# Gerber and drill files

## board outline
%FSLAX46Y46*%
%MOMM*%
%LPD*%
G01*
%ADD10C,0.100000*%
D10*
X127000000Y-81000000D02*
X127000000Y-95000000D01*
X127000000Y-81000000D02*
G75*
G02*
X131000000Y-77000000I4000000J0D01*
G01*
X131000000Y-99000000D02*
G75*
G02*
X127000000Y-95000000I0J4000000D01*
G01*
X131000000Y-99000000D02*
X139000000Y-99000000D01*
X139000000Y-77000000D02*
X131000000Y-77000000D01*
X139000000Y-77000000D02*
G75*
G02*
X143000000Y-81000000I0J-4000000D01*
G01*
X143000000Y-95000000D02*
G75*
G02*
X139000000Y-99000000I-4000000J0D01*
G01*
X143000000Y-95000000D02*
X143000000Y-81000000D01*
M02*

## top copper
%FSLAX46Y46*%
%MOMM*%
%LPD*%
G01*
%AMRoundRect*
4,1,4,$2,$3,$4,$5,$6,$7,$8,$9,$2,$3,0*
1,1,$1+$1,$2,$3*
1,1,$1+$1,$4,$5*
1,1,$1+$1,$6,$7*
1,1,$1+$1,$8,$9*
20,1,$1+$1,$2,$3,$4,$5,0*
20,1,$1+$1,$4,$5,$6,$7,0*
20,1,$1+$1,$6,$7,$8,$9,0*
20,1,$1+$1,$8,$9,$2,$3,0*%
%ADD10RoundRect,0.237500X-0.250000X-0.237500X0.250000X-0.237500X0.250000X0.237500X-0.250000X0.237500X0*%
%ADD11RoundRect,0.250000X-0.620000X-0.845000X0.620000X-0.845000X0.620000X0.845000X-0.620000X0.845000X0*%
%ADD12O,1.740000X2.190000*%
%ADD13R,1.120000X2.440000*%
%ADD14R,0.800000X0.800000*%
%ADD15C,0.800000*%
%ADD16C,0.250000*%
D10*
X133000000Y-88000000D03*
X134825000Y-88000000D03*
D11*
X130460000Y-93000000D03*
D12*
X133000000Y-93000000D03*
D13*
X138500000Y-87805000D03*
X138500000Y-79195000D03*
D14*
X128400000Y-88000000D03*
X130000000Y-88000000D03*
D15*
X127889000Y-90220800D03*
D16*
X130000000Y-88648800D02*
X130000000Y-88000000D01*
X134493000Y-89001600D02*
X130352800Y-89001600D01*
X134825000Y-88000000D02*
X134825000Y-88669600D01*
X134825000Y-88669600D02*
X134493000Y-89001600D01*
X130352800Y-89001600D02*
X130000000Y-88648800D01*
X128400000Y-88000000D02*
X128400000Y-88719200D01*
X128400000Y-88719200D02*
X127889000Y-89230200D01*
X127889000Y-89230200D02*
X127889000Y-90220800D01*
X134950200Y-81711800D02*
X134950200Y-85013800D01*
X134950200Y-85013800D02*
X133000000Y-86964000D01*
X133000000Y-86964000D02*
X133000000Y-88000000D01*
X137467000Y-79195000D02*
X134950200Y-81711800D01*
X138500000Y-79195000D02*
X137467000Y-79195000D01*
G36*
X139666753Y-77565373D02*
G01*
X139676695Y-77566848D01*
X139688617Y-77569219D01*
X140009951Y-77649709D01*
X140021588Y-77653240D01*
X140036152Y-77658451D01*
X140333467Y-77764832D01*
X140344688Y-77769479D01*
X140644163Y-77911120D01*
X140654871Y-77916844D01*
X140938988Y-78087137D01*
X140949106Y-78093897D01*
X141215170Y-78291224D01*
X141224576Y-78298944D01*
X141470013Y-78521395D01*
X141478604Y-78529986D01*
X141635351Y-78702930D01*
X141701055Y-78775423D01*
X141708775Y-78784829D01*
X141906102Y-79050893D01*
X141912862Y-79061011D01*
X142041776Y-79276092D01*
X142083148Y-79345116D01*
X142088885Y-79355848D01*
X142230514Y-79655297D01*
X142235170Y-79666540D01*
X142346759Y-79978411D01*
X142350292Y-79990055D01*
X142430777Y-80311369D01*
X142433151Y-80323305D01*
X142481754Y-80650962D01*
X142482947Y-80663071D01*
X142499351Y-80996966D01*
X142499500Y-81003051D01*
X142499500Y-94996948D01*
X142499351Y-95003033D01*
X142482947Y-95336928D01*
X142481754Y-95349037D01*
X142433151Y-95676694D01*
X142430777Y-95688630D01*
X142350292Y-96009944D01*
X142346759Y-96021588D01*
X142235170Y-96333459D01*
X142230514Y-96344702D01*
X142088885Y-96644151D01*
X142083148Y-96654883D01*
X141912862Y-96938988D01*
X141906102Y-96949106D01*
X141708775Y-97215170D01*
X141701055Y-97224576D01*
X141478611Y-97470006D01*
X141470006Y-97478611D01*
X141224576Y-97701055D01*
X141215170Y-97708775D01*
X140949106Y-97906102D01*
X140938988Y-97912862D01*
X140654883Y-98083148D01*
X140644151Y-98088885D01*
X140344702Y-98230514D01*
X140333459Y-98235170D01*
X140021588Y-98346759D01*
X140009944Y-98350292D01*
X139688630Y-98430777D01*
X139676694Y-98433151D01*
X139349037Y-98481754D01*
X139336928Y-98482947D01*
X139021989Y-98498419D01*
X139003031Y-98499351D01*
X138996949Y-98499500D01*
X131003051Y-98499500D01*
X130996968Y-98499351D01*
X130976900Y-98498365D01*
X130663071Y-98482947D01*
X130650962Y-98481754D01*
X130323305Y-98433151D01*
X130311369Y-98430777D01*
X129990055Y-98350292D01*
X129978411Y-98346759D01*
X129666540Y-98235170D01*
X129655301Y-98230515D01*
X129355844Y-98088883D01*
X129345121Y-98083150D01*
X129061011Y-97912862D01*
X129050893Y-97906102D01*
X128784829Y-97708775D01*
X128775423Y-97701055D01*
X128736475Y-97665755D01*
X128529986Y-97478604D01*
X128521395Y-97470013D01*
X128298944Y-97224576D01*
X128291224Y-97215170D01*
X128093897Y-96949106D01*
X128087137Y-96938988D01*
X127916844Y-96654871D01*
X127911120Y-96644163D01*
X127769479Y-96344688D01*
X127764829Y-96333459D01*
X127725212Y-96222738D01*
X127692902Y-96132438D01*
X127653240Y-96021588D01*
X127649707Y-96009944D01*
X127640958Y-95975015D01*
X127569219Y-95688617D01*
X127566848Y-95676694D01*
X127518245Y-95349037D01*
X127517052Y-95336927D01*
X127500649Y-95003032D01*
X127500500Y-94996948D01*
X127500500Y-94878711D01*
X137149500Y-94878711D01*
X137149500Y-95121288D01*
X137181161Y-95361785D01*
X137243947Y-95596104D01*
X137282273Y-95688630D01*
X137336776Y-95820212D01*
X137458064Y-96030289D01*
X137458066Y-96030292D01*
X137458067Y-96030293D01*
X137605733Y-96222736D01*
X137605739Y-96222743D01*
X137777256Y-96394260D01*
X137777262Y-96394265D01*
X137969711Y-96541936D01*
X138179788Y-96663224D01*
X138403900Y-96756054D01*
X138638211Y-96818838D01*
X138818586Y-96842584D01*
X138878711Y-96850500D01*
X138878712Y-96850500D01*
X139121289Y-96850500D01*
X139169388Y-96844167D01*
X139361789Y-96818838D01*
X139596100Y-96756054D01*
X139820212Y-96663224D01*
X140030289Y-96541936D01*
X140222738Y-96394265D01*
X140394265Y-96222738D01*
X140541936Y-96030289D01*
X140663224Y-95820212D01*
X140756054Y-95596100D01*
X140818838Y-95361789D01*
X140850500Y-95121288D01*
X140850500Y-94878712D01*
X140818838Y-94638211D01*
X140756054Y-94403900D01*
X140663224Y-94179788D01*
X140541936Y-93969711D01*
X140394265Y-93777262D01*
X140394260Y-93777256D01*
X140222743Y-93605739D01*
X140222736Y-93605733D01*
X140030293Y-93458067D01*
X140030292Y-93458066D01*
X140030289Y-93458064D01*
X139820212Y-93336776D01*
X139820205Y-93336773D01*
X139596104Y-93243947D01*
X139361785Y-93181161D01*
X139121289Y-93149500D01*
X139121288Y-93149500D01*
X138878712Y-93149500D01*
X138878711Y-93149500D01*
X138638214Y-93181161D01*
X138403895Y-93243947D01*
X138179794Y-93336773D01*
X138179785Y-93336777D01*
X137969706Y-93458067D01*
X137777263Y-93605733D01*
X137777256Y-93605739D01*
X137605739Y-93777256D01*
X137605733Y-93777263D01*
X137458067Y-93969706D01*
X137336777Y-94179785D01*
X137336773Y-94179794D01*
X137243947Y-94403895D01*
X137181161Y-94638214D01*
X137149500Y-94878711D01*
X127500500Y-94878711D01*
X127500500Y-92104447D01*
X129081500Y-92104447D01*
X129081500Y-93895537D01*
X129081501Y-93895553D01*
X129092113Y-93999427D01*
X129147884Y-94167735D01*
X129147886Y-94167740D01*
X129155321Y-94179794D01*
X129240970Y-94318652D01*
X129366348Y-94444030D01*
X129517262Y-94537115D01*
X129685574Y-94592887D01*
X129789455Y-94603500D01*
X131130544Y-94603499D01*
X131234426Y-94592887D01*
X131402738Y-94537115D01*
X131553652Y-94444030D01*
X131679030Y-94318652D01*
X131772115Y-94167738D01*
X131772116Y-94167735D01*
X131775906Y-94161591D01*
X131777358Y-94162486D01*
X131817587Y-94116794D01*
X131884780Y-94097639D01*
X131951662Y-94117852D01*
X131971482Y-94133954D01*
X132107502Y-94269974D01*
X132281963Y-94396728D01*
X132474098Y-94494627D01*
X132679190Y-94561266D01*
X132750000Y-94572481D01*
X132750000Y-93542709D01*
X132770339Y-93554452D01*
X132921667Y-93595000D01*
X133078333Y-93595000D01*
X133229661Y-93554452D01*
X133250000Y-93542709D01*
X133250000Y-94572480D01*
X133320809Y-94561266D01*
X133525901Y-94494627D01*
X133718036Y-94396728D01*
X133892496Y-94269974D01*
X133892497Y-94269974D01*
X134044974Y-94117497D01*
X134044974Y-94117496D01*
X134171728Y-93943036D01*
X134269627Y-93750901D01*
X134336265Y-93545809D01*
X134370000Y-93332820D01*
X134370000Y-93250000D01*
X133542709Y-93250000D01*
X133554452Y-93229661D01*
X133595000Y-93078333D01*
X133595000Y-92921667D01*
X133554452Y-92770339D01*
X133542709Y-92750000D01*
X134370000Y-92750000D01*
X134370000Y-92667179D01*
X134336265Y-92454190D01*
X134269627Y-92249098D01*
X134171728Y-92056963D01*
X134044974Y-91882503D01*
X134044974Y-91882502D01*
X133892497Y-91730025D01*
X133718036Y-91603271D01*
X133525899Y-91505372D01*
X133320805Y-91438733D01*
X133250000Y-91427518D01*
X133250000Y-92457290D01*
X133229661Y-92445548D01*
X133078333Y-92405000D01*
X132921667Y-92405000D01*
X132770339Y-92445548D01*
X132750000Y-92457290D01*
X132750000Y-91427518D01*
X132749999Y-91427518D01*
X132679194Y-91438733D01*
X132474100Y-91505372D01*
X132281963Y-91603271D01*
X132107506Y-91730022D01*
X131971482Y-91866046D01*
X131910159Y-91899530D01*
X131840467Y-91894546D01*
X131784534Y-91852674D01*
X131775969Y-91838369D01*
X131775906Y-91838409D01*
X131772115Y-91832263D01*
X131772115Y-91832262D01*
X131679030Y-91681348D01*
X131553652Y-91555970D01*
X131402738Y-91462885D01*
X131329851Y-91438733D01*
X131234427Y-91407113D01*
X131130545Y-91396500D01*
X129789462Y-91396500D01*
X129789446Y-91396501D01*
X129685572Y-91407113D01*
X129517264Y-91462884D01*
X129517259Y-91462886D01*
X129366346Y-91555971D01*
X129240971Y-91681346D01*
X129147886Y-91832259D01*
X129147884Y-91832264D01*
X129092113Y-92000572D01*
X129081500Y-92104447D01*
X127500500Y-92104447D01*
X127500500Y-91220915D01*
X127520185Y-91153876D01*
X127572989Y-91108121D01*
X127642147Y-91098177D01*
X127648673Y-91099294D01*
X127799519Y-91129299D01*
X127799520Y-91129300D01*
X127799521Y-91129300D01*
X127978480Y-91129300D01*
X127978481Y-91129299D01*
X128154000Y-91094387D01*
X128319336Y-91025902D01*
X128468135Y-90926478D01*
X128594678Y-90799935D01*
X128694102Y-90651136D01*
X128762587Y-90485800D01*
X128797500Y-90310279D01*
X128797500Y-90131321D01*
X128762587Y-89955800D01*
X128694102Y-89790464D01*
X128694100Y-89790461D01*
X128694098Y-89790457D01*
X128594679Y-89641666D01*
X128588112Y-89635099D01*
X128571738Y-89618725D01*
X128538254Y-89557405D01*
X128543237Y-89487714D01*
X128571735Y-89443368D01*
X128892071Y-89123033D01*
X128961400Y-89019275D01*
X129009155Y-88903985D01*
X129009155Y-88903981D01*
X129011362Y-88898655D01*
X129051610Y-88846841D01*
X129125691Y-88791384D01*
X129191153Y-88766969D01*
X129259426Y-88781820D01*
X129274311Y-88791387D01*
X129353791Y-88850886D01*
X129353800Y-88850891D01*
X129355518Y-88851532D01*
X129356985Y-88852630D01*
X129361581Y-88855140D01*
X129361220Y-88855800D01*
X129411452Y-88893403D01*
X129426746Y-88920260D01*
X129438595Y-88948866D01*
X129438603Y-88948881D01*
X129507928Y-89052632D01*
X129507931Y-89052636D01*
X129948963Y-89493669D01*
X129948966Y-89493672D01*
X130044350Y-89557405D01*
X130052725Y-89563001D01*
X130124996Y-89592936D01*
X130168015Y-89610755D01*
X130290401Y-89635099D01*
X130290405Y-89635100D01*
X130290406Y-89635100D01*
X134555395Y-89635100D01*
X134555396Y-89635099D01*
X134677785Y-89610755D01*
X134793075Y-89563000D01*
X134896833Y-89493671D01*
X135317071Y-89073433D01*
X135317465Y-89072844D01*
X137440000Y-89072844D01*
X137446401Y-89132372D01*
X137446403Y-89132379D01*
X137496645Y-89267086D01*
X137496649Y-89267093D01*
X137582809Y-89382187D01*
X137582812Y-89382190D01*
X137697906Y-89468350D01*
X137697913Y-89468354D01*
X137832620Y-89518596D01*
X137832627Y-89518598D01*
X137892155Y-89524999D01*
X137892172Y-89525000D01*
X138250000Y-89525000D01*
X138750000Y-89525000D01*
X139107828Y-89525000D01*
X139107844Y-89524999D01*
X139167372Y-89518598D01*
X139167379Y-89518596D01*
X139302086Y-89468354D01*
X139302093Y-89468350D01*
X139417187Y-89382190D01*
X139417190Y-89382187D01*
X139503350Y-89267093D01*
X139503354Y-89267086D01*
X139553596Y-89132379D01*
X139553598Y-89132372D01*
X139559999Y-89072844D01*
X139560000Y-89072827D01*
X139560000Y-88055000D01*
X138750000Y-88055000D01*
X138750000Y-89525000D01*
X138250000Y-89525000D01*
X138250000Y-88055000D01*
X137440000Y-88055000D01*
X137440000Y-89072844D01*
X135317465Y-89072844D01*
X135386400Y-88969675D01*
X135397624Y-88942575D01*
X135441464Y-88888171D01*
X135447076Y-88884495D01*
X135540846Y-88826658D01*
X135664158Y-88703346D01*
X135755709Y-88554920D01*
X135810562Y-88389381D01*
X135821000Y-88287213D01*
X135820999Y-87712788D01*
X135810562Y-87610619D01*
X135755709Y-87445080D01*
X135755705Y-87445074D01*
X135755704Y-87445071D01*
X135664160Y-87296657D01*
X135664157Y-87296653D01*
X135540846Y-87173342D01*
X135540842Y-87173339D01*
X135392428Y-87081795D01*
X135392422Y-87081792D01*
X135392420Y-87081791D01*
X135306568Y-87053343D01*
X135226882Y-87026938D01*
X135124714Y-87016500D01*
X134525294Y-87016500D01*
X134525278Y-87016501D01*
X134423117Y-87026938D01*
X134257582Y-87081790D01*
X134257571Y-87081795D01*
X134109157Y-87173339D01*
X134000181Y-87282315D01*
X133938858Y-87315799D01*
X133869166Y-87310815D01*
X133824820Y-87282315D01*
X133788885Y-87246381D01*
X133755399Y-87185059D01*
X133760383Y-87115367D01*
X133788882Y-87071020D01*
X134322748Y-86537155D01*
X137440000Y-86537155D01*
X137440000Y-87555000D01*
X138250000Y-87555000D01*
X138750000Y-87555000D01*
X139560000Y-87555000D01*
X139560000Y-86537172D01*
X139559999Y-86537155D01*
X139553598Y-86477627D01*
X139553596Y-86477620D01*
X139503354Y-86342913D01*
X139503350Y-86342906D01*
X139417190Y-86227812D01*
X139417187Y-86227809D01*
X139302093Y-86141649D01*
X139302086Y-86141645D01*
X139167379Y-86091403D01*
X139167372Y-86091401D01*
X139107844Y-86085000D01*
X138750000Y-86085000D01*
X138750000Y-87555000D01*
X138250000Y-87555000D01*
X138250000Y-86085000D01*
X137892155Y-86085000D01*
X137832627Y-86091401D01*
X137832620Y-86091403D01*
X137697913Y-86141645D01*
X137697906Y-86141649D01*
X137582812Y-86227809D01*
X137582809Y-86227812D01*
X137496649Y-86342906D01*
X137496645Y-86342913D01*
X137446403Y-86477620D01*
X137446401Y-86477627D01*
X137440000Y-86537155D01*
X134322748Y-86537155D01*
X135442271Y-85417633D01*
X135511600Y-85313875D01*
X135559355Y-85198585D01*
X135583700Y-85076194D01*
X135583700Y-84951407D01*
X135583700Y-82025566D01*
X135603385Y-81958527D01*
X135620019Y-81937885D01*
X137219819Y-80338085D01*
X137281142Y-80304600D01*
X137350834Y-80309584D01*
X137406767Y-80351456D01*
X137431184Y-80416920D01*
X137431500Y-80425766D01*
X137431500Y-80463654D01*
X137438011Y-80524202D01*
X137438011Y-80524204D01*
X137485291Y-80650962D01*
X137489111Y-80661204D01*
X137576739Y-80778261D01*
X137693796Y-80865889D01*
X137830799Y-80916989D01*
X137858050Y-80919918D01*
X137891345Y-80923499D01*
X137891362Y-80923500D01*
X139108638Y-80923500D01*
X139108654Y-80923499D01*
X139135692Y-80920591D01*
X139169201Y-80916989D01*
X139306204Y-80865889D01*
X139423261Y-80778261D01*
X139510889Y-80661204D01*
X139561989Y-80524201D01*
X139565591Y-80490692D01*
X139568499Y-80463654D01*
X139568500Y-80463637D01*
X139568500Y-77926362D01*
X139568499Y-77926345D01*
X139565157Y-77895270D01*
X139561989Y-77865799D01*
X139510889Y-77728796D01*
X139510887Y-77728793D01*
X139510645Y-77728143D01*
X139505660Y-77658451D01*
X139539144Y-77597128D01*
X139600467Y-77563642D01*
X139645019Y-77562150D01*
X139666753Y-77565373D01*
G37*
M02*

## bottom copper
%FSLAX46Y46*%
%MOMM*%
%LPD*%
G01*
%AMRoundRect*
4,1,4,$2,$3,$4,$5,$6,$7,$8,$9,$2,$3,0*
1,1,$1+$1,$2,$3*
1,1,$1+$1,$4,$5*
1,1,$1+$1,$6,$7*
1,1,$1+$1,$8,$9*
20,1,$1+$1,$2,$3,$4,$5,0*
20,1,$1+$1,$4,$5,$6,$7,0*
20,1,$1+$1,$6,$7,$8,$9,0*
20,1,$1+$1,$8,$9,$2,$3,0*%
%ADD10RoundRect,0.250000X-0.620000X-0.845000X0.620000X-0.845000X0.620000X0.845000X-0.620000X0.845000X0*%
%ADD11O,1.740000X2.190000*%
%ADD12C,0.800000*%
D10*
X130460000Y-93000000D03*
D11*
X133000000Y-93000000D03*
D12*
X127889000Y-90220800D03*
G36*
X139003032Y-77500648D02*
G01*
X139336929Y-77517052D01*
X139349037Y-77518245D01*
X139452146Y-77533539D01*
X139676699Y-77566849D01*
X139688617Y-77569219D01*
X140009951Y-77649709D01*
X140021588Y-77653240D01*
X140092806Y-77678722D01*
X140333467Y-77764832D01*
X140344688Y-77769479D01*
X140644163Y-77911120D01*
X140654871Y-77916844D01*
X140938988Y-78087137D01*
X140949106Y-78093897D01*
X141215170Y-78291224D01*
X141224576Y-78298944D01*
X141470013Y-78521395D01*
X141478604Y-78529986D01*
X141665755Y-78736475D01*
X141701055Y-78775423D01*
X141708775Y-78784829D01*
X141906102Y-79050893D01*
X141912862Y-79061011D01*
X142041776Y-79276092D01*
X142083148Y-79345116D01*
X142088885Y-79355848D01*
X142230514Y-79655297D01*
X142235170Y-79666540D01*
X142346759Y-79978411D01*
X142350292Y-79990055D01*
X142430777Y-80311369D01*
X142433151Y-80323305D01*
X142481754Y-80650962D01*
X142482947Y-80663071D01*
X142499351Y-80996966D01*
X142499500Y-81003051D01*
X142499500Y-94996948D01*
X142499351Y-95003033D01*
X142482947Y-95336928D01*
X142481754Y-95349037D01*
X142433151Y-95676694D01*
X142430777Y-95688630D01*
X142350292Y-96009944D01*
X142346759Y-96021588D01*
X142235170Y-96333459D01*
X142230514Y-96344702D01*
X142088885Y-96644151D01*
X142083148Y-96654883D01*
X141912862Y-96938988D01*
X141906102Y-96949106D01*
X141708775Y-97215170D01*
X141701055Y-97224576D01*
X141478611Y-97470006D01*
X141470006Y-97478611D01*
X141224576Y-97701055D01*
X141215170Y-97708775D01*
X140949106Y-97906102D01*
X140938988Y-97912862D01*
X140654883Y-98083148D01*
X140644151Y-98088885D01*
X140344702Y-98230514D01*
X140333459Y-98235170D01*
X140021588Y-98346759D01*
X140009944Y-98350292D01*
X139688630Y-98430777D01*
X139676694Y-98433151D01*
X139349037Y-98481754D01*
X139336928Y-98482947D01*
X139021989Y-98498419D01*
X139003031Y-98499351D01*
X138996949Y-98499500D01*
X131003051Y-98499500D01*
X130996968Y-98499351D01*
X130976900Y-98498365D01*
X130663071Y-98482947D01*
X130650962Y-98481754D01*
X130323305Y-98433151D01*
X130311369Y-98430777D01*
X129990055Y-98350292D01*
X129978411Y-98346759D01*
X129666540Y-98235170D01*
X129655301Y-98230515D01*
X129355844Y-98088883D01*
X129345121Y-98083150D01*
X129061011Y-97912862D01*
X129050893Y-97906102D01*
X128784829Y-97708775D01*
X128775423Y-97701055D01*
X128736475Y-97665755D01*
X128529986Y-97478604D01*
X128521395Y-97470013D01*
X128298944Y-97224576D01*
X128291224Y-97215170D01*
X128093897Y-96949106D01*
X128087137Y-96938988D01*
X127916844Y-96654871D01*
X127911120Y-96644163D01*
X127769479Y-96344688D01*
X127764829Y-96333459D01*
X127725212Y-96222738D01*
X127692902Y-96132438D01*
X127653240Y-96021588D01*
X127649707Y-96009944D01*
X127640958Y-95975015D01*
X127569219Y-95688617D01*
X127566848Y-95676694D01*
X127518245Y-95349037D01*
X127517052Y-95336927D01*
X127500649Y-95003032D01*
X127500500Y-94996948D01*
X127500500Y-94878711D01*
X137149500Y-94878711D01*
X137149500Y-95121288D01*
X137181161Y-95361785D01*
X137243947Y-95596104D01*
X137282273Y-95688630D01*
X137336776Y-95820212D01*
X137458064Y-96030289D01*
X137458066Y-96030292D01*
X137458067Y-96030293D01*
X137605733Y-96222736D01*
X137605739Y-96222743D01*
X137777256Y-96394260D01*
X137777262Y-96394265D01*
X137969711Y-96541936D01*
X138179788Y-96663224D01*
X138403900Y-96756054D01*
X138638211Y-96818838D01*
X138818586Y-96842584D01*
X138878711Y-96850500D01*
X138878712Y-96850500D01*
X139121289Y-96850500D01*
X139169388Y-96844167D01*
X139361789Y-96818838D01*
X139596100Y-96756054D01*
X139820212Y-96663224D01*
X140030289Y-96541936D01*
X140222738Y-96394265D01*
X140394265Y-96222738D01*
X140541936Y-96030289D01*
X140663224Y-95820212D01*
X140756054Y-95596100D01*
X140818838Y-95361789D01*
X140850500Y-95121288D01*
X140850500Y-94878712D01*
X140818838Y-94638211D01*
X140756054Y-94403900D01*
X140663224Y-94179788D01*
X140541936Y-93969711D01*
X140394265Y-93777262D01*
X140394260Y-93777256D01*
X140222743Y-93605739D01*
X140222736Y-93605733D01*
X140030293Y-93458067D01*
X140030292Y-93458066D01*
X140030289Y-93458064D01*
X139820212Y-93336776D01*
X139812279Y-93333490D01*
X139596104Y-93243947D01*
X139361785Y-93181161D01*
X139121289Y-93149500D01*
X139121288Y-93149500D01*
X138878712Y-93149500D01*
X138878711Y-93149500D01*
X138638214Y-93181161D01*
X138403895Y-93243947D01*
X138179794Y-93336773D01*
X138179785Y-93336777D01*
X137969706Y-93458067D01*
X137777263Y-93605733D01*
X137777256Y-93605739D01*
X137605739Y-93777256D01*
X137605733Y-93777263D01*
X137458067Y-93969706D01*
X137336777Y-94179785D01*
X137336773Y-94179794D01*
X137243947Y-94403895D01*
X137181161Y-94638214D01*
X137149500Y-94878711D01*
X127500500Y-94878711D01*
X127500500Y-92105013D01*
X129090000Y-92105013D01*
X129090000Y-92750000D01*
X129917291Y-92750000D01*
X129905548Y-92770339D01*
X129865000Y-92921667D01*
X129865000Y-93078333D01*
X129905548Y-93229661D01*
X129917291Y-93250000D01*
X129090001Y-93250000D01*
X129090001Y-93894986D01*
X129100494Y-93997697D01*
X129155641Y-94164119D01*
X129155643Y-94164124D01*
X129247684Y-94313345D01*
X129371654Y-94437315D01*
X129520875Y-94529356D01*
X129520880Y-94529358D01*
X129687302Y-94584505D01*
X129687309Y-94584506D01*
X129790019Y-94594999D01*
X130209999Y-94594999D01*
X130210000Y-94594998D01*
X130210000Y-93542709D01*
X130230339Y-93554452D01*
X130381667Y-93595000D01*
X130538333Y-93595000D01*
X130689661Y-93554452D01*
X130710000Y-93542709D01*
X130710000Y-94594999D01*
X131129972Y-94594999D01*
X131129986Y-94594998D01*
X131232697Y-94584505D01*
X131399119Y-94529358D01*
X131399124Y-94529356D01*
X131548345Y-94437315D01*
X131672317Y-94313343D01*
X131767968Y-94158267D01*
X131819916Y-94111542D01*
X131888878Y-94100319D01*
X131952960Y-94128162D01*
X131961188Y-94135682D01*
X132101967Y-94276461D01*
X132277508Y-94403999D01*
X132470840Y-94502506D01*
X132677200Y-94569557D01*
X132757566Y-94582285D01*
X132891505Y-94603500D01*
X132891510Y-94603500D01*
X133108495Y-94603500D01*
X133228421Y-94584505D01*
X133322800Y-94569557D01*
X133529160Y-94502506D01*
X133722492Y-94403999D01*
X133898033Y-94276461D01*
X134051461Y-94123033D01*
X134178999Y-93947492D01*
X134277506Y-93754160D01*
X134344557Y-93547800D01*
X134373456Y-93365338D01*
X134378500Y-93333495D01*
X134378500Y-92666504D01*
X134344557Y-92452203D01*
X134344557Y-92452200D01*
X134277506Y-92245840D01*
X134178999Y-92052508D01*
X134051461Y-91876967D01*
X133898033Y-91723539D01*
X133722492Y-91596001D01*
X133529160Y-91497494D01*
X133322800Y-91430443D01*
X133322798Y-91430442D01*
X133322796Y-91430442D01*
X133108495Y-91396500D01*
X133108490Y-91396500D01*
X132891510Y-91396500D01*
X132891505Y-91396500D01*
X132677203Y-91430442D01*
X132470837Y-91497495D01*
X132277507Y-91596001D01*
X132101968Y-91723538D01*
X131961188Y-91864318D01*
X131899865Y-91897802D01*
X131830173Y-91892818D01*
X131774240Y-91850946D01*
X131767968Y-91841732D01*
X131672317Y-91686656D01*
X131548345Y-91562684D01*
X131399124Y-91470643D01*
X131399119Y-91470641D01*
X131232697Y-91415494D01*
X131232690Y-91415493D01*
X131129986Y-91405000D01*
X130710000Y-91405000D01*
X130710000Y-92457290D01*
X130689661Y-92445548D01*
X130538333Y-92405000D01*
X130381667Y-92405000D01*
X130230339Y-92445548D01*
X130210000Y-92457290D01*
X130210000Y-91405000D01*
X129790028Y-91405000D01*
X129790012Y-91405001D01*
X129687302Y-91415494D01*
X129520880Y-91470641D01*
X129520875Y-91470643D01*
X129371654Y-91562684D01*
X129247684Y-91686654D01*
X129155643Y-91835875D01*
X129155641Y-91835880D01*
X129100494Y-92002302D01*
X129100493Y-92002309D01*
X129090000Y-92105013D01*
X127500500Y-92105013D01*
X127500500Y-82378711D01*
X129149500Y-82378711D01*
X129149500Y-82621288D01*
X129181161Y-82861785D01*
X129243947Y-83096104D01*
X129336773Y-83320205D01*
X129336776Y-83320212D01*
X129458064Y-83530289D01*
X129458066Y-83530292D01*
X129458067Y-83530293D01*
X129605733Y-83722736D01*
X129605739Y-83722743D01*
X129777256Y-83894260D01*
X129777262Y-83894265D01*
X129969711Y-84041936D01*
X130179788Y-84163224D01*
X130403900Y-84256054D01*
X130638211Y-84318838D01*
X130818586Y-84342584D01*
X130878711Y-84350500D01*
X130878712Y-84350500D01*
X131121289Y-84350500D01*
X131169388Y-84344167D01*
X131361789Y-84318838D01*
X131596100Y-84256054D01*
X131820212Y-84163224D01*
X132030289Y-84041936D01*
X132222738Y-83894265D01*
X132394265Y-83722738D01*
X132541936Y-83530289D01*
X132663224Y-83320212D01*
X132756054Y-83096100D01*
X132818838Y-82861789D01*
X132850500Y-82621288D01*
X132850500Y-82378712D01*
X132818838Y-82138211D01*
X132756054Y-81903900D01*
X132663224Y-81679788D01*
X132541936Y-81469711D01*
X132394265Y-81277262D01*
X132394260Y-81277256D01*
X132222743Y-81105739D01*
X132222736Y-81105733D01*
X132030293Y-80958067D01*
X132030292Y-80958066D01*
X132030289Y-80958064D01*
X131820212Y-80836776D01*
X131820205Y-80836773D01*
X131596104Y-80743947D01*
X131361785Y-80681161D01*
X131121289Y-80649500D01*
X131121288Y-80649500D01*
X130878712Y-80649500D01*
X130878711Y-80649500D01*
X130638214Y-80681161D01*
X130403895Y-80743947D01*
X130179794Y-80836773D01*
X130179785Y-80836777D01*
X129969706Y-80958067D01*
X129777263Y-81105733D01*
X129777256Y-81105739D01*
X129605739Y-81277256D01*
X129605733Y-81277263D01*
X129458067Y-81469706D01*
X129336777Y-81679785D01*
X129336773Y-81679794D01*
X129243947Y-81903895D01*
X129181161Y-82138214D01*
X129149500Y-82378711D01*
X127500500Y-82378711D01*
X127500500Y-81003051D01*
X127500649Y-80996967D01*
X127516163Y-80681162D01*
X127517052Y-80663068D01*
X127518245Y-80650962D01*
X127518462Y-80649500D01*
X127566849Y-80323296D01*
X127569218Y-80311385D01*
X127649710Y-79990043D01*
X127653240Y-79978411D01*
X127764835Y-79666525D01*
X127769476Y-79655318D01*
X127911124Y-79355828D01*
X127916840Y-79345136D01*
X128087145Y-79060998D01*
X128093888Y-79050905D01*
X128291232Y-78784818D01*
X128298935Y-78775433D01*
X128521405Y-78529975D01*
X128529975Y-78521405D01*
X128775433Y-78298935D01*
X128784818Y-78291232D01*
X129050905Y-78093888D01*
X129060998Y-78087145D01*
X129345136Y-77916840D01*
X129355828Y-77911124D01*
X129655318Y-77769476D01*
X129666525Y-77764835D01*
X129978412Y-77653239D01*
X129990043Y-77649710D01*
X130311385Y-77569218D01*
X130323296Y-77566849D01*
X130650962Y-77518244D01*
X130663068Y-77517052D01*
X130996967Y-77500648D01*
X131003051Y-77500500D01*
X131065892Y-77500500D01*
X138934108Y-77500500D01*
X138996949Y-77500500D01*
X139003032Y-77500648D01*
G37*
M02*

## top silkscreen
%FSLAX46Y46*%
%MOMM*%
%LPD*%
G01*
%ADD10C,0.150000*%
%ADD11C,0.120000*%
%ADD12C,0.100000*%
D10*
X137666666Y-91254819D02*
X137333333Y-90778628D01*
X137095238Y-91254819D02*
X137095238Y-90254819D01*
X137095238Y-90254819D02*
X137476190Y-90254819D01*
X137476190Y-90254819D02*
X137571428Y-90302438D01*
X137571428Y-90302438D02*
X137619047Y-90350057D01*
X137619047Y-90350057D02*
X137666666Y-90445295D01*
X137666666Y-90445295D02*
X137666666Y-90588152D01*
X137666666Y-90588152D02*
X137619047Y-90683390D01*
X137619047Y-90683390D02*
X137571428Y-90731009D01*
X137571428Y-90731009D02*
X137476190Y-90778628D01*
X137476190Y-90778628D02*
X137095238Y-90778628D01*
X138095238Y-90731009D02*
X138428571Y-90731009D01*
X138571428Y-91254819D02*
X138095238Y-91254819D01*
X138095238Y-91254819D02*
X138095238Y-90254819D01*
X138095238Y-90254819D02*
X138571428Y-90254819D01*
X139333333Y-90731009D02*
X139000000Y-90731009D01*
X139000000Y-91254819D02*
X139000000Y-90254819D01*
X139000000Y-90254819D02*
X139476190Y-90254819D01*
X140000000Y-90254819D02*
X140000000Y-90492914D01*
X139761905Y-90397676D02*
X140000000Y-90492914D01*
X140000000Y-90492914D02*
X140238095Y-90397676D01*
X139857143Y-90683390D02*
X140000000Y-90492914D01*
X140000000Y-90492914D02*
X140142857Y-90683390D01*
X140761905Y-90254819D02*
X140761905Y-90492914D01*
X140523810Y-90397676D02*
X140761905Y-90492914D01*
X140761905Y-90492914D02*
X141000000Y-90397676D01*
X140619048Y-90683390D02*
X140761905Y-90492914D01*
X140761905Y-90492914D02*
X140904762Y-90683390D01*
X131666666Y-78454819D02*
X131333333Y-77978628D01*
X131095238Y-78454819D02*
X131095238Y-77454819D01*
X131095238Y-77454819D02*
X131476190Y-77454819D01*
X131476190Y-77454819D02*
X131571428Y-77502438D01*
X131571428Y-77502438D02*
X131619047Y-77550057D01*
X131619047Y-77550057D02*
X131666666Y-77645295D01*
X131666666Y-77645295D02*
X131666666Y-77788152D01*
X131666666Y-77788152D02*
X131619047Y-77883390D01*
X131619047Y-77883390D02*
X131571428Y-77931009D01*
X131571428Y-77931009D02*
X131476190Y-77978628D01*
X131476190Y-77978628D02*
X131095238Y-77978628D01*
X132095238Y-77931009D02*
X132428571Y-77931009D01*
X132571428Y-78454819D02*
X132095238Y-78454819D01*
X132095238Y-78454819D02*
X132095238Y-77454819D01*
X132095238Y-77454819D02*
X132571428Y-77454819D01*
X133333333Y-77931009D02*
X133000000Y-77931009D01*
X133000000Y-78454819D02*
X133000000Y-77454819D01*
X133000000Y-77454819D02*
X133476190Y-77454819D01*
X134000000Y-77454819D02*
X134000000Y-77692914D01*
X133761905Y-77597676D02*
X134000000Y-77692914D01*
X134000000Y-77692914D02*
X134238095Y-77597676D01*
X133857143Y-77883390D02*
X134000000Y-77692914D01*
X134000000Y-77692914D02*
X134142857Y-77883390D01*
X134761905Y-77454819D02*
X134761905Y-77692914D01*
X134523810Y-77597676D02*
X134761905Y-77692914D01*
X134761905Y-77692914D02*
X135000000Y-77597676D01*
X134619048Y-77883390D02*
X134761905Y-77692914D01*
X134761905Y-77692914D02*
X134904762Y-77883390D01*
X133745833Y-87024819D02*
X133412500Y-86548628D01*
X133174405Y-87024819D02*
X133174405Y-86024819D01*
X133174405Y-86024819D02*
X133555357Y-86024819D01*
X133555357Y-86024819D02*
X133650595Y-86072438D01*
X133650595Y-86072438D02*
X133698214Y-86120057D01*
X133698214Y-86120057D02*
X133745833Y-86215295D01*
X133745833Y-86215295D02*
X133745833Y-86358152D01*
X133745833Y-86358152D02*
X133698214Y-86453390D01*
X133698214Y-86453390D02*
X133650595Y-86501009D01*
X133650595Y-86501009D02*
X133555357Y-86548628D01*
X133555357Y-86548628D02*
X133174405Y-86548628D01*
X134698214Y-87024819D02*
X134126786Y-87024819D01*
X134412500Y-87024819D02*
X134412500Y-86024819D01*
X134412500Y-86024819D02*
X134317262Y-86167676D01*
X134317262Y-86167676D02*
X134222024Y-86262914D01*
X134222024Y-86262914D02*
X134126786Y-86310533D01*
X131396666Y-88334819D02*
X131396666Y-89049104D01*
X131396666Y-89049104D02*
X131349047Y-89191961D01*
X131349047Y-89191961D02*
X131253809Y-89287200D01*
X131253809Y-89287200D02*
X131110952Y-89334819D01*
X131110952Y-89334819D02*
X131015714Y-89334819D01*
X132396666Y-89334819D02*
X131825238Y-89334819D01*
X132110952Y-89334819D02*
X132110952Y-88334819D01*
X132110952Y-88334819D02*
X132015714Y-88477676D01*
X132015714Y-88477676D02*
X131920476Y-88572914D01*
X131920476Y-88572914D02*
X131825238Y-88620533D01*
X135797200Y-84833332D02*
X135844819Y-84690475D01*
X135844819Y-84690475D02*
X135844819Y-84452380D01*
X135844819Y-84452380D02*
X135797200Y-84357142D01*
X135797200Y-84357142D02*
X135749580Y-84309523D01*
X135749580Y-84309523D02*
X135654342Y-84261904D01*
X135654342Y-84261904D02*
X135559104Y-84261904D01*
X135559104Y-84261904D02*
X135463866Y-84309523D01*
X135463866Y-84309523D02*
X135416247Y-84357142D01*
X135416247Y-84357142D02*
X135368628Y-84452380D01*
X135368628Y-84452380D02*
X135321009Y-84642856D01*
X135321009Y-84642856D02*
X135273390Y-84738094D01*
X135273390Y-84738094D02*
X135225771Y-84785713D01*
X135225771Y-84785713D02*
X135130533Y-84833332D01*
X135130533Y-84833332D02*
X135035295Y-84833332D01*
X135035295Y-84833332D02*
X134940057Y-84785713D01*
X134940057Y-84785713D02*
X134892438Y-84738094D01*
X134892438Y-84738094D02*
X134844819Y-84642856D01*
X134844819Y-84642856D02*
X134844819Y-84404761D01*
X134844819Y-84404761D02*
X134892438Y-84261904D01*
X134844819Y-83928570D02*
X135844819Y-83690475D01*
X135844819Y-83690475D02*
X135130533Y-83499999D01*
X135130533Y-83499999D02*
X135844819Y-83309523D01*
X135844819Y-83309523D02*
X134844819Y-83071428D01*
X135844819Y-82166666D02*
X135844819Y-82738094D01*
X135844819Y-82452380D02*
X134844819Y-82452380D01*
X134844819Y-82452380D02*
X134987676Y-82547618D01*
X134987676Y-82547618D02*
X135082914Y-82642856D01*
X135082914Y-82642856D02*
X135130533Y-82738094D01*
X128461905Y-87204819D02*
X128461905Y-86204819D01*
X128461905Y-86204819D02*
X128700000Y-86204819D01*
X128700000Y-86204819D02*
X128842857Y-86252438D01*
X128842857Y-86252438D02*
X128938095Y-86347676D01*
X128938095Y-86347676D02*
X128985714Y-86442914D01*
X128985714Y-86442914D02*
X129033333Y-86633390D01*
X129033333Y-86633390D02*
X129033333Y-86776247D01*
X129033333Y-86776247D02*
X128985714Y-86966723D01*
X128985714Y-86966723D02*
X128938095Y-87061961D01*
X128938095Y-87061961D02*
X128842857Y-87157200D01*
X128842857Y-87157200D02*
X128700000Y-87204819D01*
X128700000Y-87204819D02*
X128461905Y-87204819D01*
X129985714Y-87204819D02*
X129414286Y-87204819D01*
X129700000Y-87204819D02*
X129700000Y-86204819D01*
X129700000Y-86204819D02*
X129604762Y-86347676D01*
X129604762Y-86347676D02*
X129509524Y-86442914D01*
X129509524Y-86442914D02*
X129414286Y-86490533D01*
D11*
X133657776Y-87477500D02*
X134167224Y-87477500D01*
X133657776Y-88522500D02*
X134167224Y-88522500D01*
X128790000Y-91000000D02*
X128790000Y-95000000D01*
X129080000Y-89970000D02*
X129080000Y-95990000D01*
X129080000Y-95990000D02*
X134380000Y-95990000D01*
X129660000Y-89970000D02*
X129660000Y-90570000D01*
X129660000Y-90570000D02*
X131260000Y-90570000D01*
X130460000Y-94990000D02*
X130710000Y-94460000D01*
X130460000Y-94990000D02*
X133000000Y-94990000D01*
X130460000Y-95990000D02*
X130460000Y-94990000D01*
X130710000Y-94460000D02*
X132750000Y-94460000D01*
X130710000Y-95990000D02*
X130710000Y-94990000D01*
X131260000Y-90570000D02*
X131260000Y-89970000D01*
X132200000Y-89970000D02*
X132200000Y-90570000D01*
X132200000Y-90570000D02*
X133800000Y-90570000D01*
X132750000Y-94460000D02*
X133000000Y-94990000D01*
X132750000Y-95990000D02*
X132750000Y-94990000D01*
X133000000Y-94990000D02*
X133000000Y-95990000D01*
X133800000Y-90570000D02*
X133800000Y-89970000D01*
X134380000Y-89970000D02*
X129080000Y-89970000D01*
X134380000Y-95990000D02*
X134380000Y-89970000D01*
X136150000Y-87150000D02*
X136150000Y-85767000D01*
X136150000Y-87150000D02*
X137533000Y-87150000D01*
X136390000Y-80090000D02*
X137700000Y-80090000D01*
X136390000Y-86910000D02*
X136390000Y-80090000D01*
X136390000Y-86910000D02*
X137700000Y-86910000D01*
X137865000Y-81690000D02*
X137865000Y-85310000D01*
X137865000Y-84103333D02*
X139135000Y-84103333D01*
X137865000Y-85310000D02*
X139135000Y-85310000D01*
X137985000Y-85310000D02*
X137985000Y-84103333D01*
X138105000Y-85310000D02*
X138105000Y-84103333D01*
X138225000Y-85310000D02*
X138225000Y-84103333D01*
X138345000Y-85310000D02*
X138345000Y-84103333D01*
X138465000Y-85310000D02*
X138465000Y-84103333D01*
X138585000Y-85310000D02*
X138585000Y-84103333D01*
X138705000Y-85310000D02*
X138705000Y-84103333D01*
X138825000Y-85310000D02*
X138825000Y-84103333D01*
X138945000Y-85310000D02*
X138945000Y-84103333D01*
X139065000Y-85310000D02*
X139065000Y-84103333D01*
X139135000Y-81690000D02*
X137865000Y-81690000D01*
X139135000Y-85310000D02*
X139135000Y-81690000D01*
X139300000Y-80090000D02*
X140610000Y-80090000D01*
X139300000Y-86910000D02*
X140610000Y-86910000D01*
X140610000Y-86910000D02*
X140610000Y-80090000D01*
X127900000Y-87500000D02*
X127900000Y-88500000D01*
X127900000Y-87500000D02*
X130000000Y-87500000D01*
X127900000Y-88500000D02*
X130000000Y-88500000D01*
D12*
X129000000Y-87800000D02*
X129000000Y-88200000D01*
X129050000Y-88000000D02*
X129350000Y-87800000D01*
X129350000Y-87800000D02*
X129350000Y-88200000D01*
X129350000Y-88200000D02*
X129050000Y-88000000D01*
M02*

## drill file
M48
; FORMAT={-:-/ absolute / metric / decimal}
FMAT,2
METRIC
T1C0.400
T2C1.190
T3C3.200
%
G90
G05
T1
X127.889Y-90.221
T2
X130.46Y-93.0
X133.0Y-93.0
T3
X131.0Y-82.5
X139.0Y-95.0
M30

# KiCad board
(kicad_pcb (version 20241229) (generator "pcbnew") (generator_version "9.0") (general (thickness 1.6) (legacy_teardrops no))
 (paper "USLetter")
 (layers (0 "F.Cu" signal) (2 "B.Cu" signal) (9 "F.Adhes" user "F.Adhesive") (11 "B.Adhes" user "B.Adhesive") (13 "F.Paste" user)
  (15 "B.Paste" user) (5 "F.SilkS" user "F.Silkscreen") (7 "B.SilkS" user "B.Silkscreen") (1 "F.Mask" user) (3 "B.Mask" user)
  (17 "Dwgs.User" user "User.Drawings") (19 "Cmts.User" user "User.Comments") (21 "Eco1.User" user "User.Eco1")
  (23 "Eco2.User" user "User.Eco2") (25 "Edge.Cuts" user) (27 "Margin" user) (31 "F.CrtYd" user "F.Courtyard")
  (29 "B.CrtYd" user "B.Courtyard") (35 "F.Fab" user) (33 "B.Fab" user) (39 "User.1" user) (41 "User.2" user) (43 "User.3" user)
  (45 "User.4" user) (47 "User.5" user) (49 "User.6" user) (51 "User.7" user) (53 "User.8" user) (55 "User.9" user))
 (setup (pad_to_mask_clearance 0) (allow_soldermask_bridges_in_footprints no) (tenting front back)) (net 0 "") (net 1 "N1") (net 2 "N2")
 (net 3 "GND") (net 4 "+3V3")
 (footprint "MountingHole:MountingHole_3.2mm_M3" (layer "F.Cu") (at 139 95)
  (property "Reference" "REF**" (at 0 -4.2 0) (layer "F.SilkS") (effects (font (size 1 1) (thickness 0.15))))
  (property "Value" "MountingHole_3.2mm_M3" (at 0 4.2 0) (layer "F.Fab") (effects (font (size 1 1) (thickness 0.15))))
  (pad "" np_thru_hole circle (at 0 0) (size 3.2 3.2) (drill 3.2) (layers "*.Cu" "*.Mask")))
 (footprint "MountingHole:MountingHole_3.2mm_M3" (layer "F.Cu") (at 131 82.5)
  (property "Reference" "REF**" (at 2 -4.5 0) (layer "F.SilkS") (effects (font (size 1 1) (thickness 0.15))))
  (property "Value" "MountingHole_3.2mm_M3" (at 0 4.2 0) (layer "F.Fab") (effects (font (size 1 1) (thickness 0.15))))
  (pad "" np_thru_hole circle (at 0 0) (size 3.2 3.2) (drill 3.2) (layers "*.Cu" "*.Mask")))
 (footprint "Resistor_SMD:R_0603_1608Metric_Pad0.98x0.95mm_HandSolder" (layer "F.Cu") (at 133.9125 88)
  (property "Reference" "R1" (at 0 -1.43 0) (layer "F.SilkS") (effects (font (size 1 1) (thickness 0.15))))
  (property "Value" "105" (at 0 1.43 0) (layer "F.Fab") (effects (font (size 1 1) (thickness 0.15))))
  (fp_line (start -0.254724 -0.5225) (end 0.254724 -0.5225) (stroke (width 0.12) (type solid)) (layer "F.SilkS"))
  (fp_line (start -0.254724 0.5225) (end 0.254724 0.5225) (stroke (width 0.12) (type solid)) (layer "F.SilkS"))
  (pad "1" smd roundrect (at -0.9125 0) (size 0.975 0.95) (layers "F.Cu" "F.Mask" "F.Paste") (roundrect_rratio 0.25) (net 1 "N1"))
  (pad "2" smd roundrect (at 0.9125 0) (size 0.975 0.95) (layers "F.Cu" "F.Mask" "F.Paste") (roundrect_rratio 0.25) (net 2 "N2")))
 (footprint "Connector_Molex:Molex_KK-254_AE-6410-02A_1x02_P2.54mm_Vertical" (layer "F.Cu") (at 130.46 93)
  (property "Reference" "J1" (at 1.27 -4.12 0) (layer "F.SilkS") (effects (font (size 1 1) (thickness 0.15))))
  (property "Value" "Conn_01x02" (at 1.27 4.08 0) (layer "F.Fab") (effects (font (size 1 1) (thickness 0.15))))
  (fp_line (start -1.67 -2) (end -1.67 2) (stroke (width 0.12) (type solid)) (layer "F.SilkS"))
  (fp_line (start -1.38 -3.03) (end -1.38 2.99) (stroke (width 0.12) (type solid)) (layer "F.SilkS"))
  (fp_line (start -1.38 2.99) (end 3.92 2.99) (stroke (width 0.12) (type solid)) (layer "F.SilkS"))
  (fp_line (start -0.8 -3.03) (end -0.8 -2.43) (stroke (width 0.12) (type solid)) (layer "F.SilkS"))
  (fp_line (start -0.8 -2.43) (end 0.8 -2.43) (stroke (width 0.12) (type solid)) (layer "F.SilkS"))
  (fp_line (start 0 1.99) (end 0.25 1.46) (stroke (width 0.12) (type solid)) (layer "F.SilkS"))
  (fp_line (start 0 1.99) (end 2.54 1.99) (stroke (width 0.12) (type solid)) (layer "F.SilkS"))
  (fp_line (start 0 2.99) (end 0 1.99) (stroke (width 0.12) (type solid)) (layer "F.SilkS"))
  (fp_line (start 0.25 1.46) (end 2.29 1.46) (stroke (width 0.12) (type solid)) (layer "F.SilkS"))
  (fp_line (start 0.25 2.99) (end 0.25 1.99) (stroke (width 0.12) (type solid)) (layer "F.SilkS"))
  (fp_line (start 0.8 -2.43) (end 0.8 -3.03) (stroke (width 0.12) (type solid)) (layer "F.SilkS"))
  (fp_line (start 1.74 -3.03) (end 1.74 -2.43) (stroke (width 0.12) (type solid)) (layer "F.SilkS"))
  (fp_line (start 1.74 -2.43) (end 3.34 -2.43) (stroke (width 0.12) (type solid)) (layer "F.SilkS"))
  (fp_line (start 2.29 1.46) (end 2.54 1.99) (stroke (width 0.12) (type solid)) (layer "F.SilkS"))
  (fp_line (start 2.29 2.99) (end 2.29 1.99) (stroke (width 0.12) (type solid)) (layer "F.SilkS"))
  (fp_line (start 2.54 1.99) (end 2.54 2.99) (stroke (width 0.12) (type solid)) (layer "F.SilkS"))
  (fp_line (start 3.34 -2.43) (end 3.34 -3.03) (stroke (width 0.12) (type solid)) (layer "F.SilkS"))
  (fp_line (start 3.92 -3.03) (end -1.38 -3.03) (stroke (width 0.12) (type solid)) (layer "F.SilkS"))
  (fp_line (start 3.92 2.99) (end 3.92 -3.03) (stroke (width 0.12) (type solid)) (layer "F.SilkS"))
  (pad "1" thru_hole roundrect (at 0 0) (size 1.74 2.19) (drill 1.19) (layers "*.Cu" "*.Mask") (remove_unused_layers no)
   (roundrect_rratio 0.143678) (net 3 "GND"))
  (pad "2" thru_hole oval (at 2.54 0) (size 1.74 2.19) (drill 1.19) (layers "*.Cu" "*.Mask") (remove_unused_layers no) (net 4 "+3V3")))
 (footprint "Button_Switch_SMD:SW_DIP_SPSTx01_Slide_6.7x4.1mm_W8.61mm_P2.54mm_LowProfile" (layer "F.Cu") (at 138.5 83.5 90)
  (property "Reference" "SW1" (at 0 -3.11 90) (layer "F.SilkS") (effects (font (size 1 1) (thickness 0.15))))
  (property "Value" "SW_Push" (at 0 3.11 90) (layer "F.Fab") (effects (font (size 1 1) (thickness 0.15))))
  (fp_line (start -3.65 -2.35) (end -2.267 -2.35) (stroke (width 0.12) (type solid)) (layer "F.SilkS"))
  (fp_line (start -3.65 -2.35) (end -3.65 -0.967) (stroke (width 0.12) (type solid)) (layer "F.SilkS"))
  (fp_line (start 3.41 -2.11) (end 3.41 -0.8) (stroke (width 0.12) (type solid)) (layer "F.SilkS"))
  (fp_line (start -3.41 -2.11) (end 3.41 -2.11) (stroke (width 0.12) (type solid)) (layer "F.SilkS"))
  (fp_line (start -3.41 -2.11) (end -3.41 -0.8) (stroke (width 0.12) (type solid)) (layer "F.SilkS"))
  (fp_line (start 1.81 -0.635) (end -1.81 -0.635) (stroke (width 0.12) (type solid)) (layer "F.SilkS"))
  (fp_line (start -0.603333 -0.635) (end -0.603333 0.635) (stroke (width 0.12) (type solid)) (layer "F.SilkS"))
  (fp_line (start -1.81 -0.635) (end -1.81 0.635) (stroke (width 0.12) (type solid)) (layer "F.SilkS"))
  (fp_line (start -1.81 -0.515) (end -0.603333 -0.515) (stroke (width 0.12) (type solid)) (layer "F.SilkS"))
  (fp_line (start -1.81 -0.395) (end -0.603333 -0.395) (stroke (width 0.12) (type solid)) (layer "F.SilkS"))
  (fp_line (start -1.81 -0.275) (end -0.603333 -0.275) (stroke (width 0.12) (type solid)) (layer "F.SilkS"))
  (fp_line (start -1.81 -0.155) (end -0.603333 -0.155) (stroke (width 0.12) (type solid)) (layer "F.SilkS"))
  (fp_line (start -1.81 -0.035) (end -0.603333 -0.035) (stroke (width 0.12) (type solid)) (layer "F.SilkS"))
  (fp_line (start -1.81 0.085) (end -0.603333 0.085) (stroke (width 0.12) (type solid)) (layer "F.SilkS"))
  (fp_line (start -1.81 0.205) (end -0.603333 0.205) (stroke (width 0.12) (type solid)) (layer "F.SilkS"))
  (fp_line (start -1.81 0.325) (end -0.603333 0.325) (stroke (width 0.12) (type solid)) (layer "F.SilkS"))
  (fp_line (start -1.81 0.445) (end -0.603333 0.445) (stroke (width 0.12) (type solid)) (layer "F.SilkS"))
  (fp_line (start -1.81 0.565) (end -0.603333 0.565) (stroke (width 0.12) (type solid)) (layer "F.SilkS"))
  (fp_line (start 1.81 0.635) (end 1.81 -0.635) (stroke (width 0.12) (type solid)) (layer "F.SilkS"))
  (fp_line (start -1.81 0.635) (end 1.81 0.635) (stroke (width 0.12) (type solid)) (layer "F.SilkS"))
  (fp_line (start 3.41 0.8) (end 3.41 2.11) (stroke (width 0.12) (type solid)) (layer "F.SilkS"))
  (fp_line (start -3.41 0.8) (end -3.41 2.11) (stroke (width 0.12) (type solid)) (layer "F.SilkS"))
  (fp_line (start -3.41 2.11) (end 3.41 2.11) (stroke (width 0.12) (type solid)) (layer "F.SilkS"))
  (pad "1" smd rect (at -4.305 0 90) (size 2.44 1.12) (layers "F.Cu" "F.Mask" "F.Paste") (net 4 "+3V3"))
  (pad "2" smd rect (at 4.305 0 90) (size 2.44 1.12) (layers "F.Cu" "F.Mask" "F.Paste") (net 1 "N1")))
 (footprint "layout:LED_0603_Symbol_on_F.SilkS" (layer "F.Cu") (at 129.2 88)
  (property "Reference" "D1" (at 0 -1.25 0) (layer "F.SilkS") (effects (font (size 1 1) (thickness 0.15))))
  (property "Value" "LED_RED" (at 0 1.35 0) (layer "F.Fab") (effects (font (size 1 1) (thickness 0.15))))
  (fp_line (start -1.3 -0.5) (end -1.3 0.5) (stroke (width 0.12) (type solid)) (layer "F.SilkS"))
  (fp_line (start -1.3 -0.5) (end 0.8 -0.5) (stroke (width 0.12) (type solid)) (layer "F.SilkS"))
  (fp_line (start -1.3 0.5) (end 0.8 0.5) (stroke (width 0.12) (type solid)) (layer "F.SilkS"))
  (fp_line (start -0.2 -0.2) (end -0.2 0.2) (stroke (width 0.1) (type solid)) (layer "F.SilkS"))
  (fp_line (start -0.15 0) (end 0.15 -0.2) (stroke (width 0.1) (type solid)) (layer "F.SilkS"))
  (fp_line (start 0.15 -0.2) (end 0.15 0.2) (stroke (width 0.1) (type solid)) (layer "F.SilkS"))
  (fp_line (start 0.15 0.2) (end -0.15 0) (stroke (width 0.1) (type solid)) (layer "F.SilkS"))
  (pad "1" smd rect (at -0.8 0 180) (size 0.8 0.8) (layers "F.Cu" "F.Mask" "F.Paste") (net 3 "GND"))
  (pad "2" smd rect (at 0.8 0 180) (size 0.8 0.8) (layers "F.Cu" "F.Mask" "F.Paste") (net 2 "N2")))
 (gr_line (start 127 81) (end 127 95) (stroke (width 0.1) (type default)) (layer "Edge.Cuts"))
 (gr_arc (start 127 81) (mid 128.171573 78.171573) (end 131 77) (stroke (width 0.1) (type default)) (layer "Edge.Cuts"))
 (gr_arc (start 131 99) (mid 128.171573 97.828427) (end 127 95) (stroke (width 0.1) (type default)) (layer "Edge.Cuts"))
 (gr_line (start 131 99) (end 139 99) (stroke (width 0.1) (type default)) (layer "Edge.Cuts"))
 (gr_line (start 139 77) (end 131 77) (stroke (width 0.1) (type default)) (layer "Edge.Cuts"))
 (gr_arc (start 139 77) (mid 141.828427 78.171573) (end 143 81) (stroke (width 0.1) (type default)) (layer "Edge.Cuts"))
 (gr_arc (start 143 95) (mid 141.828427 97.828427) (end 139 99) (stroke (width 0.1) (type default)) (layer "Edge.Cuts"))
 (gr_line (start 143 95) (end 143 81) (stroke (width 0.1) (type default)) (layer "Edge.Cuts"))
 (segment (start 130 88.6488) (end 130 88) (width 0.25) (layer "F.Cu") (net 2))
 (segment (start 134.493 89.0016) (end 130.3528 89.0016) (width 0.25) (layer "F.Cu") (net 2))
 (segment (start 134.825 88) (end 134.825 88.6696) (width 0.25) (layer "F.Cu") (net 2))
 (segment (start 134.825 88.6696) (end 134.493 89.0016) (width 0.25) (layer "F.Cu") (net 2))
 (segment (start 130.3528 89.0016) (end 130 88.6488) (width 0.25) (layer "F.Cu") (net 2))
 (segment (start 128.4 88) (end 128.4 88.7192) (width 0.25) (layer "F.Cu") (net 3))
 (segment (start 128.4 88.7192) (end 127.889 89.2302) (width 0.25) (layer "F.Cu") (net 3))
 (segment (start 127.889 89.2302) (end 127.889 90.2208) (width 0.25) (layer "F.Cu") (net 3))
 (via (at 127.889 90.2208) (size 0.8) (drill 0.4) (layers "F.Cu" "B.Cu") (free yes) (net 3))
 (segment (start 134.9502 81.7118) (end 134.9502 85.0138) (width 0.25) (layer "F.Cu") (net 1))
 (segment (start 134.9502 85.0138) (end 133 86.964) (width 0.25) (layer "F.Cu") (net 1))
 (segment (start 133 86.964) (end 133 88) (width 0.25) (layer "F.Cu") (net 1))
 (segment (start 137.467 79.195) (end 134.9502 81.7118) (width 0.25) (layer "F.Cu") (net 1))
 (segment (start 138.5 79.195) (end 137.467 79.195) (width 0.25) (layer "F.Cu") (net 1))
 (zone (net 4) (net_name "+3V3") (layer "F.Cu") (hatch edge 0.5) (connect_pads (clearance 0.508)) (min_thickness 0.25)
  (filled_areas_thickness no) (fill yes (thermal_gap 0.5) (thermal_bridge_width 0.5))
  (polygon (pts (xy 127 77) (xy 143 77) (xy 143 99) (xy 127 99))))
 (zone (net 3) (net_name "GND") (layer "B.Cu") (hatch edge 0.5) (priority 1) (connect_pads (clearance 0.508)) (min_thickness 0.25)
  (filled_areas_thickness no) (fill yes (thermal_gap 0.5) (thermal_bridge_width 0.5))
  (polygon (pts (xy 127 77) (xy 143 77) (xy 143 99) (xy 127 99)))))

